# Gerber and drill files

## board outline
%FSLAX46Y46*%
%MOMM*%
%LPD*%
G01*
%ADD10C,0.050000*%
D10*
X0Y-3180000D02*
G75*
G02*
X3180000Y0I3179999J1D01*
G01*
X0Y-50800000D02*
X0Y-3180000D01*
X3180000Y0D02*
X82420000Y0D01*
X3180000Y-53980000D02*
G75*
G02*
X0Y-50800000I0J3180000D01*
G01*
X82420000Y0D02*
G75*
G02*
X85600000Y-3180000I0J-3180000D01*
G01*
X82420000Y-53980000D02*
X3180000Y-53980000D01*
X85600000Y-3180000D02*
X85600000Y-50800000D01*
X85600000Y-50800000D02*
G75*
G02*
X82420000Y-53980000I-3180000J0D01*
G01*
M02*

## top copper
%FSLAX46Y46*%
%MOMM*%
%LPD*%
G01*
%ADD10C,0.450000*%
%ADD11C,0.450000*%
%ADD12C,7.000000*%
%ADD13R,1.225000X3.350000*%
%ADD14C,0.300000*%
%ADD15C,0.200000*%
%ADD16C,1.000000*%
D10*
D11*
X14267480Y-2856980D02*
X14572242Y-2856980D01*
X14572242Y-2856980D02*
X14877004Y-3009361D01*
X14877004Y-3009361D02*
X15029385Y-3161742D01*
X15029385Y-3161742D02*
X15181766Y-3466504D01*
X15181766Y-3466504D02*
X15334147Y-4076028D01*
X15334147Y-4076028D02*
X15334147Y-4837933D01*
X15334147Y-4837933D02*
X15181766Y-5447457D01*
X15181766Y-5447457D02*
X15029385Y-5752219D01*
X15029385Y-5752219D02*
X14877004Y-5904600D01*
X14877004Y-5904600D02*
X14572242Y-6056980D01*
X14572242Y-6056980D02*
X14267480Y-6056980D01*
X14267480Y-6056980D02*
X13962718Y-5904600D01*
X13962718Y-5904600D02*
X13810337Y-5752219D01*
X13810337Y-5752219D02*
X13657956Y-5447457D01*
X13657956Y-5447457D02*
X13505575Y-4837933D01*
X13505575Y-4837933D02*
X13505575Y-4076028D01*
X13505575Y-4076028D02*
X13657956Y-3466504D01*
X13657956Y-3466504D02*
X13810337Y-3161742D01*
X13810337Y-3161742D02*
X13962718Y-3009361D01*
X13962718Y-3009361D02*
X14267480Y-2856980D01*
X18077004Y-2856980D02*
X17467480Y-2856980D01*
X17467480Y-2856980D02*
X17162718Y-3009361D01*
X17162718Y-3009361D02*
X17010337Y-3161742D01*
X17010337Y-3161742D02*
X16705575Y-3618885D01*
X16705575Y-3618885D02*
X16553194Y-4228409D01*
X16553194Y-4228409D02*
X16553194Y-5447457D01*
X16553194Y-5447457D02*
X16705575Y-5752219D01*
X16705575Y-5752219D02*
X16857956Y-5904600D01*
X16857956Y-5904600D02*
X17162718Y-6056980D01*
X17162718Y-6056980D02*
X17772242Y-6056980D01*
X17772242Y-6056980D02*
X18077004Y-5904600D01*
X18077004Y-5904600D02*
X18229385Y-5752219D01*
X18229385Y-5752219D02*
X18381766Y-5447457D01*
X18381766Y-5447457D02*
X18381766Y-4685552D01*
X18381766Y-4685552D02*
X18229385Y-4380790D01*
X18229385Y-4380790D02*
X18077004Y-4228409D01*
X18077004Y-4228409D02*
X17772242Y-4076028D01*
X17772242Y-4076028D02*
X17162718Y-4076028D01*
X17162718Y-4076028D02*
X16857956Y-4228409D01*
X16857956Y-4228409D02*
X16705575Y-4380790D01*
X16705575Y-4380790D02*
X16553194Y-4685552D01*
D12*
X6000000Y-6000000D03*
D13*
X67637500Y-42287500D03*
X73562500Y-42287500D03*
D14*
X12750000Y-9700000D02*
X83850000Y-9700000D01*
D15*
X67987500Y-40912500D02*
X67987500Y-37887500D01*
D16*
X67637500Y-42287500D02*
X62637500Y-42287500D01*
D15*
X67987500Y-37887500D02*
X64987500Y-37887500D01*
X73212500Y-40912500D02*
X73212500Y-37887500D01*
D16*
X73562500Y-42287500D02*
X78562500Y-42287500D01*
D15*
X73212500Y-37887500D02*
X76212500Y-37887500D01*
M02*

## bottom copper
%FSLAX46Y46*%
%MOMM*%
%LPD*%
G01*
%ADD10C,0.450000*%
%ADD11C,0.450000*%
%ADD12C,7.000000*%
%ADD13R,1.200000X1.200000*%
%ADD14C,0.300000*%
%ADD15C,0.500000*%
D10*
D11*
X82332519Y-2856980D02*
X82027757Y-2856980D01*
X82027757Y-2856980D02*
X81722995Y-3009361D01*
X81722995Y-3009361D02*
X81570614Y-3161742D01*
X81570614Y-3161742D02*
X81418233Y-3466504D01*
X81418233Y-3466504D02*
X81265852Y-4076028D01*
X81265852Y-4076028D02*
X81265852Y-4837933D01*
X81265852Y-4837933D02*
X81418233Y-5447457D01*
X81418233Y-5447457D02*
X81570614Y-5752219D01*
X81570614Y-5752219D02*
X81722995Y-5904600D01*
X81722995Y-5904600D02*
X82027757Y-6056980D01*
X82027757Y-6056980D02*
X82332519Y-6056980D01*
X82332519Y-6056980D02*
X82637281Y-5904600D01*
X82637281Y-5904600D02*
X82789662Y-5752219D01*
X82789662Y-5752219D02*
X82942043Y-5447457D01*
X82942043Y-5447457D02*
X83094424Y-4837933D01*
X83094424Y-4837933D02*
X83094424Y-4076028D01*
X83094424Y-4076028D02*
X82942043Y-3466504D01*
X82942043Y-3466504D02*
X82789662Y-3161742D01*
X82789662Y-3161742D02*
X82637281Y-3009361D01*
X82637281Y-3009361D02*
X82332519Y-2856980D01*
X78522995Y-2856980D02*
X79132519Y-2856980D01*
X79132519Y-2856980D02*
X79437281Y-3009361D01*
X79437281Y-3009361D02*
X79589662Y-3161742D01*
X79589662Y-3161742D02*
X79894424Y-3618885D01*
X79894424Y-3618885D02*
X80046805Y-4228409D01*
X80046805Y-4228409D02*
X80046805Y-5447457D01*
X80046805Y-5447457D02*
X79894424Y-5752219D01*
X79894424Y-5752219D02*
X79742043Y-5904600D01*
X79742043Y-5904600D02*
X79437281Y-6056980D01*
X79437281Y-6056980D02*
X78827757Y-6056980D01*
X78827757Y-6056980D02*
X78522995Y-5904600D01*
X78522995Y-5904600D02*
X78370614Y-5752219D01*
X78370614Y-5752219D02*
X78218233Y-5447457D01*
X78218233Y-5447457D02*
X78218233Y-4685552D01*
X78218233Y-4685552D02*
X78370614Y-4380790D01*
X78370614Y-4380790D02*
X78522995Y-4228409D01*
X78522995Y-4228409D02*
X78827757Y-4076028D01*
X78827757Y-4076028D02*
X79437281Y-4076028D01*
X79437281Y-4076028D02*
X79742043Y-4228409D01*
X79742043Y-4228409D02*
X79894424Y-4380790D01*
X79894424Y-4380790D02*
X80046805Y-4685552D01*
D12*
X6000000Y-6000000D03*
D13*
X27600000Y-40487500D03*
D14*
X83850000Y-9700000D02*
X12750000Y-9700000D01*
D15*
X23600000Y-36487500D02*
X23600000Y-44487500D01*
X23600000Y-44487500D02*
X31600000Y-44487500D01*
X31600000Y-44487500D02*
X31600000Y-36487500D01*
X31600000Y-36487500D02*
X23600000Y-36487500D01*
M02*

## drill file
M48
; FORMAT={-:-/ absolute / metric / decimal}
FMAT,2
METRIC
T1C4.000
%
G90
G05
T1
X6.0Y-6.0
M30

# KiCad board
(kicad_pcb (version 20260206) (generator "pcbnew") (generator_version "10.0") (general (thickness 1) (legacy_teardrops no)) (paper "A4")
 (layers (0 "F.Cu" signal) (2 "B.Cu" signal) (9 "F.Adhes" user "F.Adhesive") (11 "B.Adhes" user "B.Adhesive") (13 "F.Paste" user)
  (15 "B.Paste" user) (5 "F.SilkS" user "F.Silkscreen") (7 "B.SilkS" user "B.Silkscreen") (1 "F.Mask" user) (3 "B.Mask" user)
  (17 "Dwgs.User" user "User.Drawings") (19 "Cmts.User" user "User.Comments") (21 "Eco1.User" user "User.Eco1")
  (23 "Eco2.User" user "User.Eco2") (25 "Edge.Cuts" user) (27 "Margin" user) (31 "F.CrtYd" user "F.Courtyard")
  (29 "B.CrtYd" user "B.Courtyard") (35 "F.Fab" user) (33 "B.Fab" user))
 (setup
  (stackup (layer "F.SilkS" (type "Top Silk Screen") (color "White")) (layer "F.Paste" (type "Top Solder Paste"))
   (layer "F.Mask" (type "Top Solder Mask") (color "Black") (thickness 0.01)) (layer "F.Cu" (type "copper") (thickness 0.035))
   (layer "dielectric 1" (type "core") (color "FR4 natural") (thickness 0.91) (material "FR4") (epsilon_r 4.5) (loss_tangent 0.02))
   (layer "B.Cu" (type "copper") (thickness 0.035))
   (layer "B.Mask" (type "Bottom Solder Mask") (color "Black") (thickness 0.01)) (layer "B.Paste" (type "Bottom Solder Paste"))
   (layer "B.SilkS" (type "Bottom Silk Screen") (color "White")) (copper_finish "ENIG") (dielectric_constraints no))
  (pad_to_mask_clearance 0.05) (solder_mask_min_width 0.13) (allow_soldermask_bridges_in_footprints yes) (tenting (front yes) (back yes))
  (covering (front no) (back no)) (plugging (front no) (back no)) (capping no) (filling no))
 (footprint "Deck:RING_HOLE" (layer "F.Cu") (at 6 6)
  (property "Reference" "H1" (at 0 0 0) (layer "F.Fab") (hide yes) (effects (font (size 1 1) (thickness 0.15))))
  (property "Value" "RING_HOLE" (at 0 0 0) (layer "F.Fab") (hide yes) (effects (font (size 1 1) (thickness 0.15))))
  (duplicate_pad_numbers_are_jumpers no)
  (pad "" thru_hole circle (at 0 0) (size 7 7) (drill 4) (layers "*.Cu" "*.Mask") (remove_unused_layers no)))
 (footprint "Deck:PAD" (layer "F.Cu") (at 67.6375 42.2875)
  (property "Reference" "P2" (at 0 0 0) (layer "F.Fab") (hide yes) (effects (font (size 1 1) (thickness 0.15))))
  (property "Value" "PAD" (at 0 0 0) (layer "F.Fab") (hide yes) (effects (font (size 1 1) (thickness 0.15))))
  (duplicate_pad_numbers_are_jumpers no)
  (pad "1" smd rect (at 0 0) (size 1.225 3.35) (layers "F.Cu" "F.Mask") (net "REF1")))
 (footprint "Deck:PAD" (layer "F.Cu") (at 73.5625 42.2875)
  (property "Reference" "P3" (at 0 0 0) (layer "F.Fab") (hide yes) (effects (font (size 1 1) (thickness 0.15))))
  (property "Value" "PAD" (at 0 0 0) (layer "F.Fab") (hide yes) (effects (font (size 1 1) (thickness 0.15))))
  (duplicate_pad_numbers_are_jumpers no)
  (pad "1" smd rect (at 0 0) (size 1.225 3.35) (layers "F.Cu" "F.Mask") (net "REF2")))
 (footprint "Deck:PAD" (layer "B.Cu") (at 27.6 40.4875)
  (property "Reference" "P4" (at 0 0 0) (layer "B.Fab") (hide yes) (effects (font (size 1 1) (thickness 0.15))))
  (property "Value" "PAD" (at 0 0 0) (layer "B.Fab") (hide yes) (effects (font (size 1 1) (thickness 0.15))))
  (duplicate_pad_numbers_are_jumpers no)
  (pad "1" smd rect (at 0 0) (size 1.2 1.2) (layers "B.Cu" "B.Mask") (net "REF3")))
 (gr_arc (start 0 3.18) (mid 0.9314 0.9314) (end 3.18 0) (stroke (width 0.05) (type solid)) (layer "Edge.Cuts"))
 (gr_line (start 0 50.8) (end 0 3.18) (stroke (width 0.05) (type solid)) (layer "Edge.Cuts"))
 (gr_line (start 3.18 0) (end 82.42 0) (stroke (width 0.05) (type solid)) (layer "Edge.Cuts"))
 (gr_arc (start 3.18 53.98) (mid 0.9314 53.0486) (end 0 50.8) (stroke (width 0.05) (type solid)) (layer "Edge.Cuts"))
 (gr_arc (start 82.42 0) (mid 84.6686 0.9314) (end 85.6 3.18) (stroke (width 0.05) (type solid)) (layer "Edge.Cuts"))
 (gr_line (start 82.42 53.98) (end 3.18 53.98) (stroke (width 0.05) (type solid)) (layer "Edge.Cuts"))
 (gr_line (start 85.6 3.18) (end 85.6 50.8) (stroke (width 0.05) (type solid)) (layer "Edge.Cuts"))
 (gr_arc (start 85.6 50.8) (mid 84.6686 53.0486) (end 82.42 53.98) (stroke (width 0.05) (type solid)) (layer "Edge.Cuts"))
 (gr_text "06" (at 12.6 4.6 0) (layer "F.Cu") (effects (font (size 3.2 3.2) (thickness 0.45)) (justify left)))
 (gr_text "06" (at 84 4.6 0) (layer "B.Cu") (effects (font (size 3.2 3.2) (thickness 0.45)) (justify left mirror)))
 (segment (start 12.75 9.7) (end 83.85 9.7) (width 0.3) (layer "F.Cu") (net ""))
 (segment (start 83.85 9.7) (end 12.75 9.7) (width 0.3) (layer "B.Cu") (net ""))
 (segment (start 67.9875 40.9125) (end 67.9875 37.8875) (width 0.2) (layer "F.Cu") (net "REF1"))
 (segment (start 67.6375 42.2875) (end 62.6375 42.2875) (width 1) (layer "F.Cu") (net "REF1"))
 (segment (start 67.9875 37.8875) (end 64.9875 37.8875) (width 0.2) (layer "F.Cu") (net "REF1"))
 (segment (start 73.2125 40.9125) (end 73.2125 37.8875) (width 0.2) (layer "F.Cu") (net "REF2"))
 (segment (start 73.5625 42.2875) (end 78.5625 42.2875) (width 1) (layer "F.Cu") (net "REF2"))
 (segment (start 73.2125 37.8875) (end 76.2125 37.8875) (width 0.2) (layer "F.Cu") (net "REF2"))
 (segment (start 23.6 36.4875) (end 23.6 44.4875) (width 0.5) (layer "B.Cu") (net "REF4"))
 (segment (start 23.6 44.4875) (end 31.6 44.4875) (width 0.5) (layer "B.Cu") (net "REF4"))
 (segment (start 31.6 44.4875) (end 31.6 36.4875) (width 0.5) (layer "B.Cu") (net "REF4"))
 (segment (start 31.6 36.4875) (end 23.6 36.4875) (width 0.5) (layer "B.Cu") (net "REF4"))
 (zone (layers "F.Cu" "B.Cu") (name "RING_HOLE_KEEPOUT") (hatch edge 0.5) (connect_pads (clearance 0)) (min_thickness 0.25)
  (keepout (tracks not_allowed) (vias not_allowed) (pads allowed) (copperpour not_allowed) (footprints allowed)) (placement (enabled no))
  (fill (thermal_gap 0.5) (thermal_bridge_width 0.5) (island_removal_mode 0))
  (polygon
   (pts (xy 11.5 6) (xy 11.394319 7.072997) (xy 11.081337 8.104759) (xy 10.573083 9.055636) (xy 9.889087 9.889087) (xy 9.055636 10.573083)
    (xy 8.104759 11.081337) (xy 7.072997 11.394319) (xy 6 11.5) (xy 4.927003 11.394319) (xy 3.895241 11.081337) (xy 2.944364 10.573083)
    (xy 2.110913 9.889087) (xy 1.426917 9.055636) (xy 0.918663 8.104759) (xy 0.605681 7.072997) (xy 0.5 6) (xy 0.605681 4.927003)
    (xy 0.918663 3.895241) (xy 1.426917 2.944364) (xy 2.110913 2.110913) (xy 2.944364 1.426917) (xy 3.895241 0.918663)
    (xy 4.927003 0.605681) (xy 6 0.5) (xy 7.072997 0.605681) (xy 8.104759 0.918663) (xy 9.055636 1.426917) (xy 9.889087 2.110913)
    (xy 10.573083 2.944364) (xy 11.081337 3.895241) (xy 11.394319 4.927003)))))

